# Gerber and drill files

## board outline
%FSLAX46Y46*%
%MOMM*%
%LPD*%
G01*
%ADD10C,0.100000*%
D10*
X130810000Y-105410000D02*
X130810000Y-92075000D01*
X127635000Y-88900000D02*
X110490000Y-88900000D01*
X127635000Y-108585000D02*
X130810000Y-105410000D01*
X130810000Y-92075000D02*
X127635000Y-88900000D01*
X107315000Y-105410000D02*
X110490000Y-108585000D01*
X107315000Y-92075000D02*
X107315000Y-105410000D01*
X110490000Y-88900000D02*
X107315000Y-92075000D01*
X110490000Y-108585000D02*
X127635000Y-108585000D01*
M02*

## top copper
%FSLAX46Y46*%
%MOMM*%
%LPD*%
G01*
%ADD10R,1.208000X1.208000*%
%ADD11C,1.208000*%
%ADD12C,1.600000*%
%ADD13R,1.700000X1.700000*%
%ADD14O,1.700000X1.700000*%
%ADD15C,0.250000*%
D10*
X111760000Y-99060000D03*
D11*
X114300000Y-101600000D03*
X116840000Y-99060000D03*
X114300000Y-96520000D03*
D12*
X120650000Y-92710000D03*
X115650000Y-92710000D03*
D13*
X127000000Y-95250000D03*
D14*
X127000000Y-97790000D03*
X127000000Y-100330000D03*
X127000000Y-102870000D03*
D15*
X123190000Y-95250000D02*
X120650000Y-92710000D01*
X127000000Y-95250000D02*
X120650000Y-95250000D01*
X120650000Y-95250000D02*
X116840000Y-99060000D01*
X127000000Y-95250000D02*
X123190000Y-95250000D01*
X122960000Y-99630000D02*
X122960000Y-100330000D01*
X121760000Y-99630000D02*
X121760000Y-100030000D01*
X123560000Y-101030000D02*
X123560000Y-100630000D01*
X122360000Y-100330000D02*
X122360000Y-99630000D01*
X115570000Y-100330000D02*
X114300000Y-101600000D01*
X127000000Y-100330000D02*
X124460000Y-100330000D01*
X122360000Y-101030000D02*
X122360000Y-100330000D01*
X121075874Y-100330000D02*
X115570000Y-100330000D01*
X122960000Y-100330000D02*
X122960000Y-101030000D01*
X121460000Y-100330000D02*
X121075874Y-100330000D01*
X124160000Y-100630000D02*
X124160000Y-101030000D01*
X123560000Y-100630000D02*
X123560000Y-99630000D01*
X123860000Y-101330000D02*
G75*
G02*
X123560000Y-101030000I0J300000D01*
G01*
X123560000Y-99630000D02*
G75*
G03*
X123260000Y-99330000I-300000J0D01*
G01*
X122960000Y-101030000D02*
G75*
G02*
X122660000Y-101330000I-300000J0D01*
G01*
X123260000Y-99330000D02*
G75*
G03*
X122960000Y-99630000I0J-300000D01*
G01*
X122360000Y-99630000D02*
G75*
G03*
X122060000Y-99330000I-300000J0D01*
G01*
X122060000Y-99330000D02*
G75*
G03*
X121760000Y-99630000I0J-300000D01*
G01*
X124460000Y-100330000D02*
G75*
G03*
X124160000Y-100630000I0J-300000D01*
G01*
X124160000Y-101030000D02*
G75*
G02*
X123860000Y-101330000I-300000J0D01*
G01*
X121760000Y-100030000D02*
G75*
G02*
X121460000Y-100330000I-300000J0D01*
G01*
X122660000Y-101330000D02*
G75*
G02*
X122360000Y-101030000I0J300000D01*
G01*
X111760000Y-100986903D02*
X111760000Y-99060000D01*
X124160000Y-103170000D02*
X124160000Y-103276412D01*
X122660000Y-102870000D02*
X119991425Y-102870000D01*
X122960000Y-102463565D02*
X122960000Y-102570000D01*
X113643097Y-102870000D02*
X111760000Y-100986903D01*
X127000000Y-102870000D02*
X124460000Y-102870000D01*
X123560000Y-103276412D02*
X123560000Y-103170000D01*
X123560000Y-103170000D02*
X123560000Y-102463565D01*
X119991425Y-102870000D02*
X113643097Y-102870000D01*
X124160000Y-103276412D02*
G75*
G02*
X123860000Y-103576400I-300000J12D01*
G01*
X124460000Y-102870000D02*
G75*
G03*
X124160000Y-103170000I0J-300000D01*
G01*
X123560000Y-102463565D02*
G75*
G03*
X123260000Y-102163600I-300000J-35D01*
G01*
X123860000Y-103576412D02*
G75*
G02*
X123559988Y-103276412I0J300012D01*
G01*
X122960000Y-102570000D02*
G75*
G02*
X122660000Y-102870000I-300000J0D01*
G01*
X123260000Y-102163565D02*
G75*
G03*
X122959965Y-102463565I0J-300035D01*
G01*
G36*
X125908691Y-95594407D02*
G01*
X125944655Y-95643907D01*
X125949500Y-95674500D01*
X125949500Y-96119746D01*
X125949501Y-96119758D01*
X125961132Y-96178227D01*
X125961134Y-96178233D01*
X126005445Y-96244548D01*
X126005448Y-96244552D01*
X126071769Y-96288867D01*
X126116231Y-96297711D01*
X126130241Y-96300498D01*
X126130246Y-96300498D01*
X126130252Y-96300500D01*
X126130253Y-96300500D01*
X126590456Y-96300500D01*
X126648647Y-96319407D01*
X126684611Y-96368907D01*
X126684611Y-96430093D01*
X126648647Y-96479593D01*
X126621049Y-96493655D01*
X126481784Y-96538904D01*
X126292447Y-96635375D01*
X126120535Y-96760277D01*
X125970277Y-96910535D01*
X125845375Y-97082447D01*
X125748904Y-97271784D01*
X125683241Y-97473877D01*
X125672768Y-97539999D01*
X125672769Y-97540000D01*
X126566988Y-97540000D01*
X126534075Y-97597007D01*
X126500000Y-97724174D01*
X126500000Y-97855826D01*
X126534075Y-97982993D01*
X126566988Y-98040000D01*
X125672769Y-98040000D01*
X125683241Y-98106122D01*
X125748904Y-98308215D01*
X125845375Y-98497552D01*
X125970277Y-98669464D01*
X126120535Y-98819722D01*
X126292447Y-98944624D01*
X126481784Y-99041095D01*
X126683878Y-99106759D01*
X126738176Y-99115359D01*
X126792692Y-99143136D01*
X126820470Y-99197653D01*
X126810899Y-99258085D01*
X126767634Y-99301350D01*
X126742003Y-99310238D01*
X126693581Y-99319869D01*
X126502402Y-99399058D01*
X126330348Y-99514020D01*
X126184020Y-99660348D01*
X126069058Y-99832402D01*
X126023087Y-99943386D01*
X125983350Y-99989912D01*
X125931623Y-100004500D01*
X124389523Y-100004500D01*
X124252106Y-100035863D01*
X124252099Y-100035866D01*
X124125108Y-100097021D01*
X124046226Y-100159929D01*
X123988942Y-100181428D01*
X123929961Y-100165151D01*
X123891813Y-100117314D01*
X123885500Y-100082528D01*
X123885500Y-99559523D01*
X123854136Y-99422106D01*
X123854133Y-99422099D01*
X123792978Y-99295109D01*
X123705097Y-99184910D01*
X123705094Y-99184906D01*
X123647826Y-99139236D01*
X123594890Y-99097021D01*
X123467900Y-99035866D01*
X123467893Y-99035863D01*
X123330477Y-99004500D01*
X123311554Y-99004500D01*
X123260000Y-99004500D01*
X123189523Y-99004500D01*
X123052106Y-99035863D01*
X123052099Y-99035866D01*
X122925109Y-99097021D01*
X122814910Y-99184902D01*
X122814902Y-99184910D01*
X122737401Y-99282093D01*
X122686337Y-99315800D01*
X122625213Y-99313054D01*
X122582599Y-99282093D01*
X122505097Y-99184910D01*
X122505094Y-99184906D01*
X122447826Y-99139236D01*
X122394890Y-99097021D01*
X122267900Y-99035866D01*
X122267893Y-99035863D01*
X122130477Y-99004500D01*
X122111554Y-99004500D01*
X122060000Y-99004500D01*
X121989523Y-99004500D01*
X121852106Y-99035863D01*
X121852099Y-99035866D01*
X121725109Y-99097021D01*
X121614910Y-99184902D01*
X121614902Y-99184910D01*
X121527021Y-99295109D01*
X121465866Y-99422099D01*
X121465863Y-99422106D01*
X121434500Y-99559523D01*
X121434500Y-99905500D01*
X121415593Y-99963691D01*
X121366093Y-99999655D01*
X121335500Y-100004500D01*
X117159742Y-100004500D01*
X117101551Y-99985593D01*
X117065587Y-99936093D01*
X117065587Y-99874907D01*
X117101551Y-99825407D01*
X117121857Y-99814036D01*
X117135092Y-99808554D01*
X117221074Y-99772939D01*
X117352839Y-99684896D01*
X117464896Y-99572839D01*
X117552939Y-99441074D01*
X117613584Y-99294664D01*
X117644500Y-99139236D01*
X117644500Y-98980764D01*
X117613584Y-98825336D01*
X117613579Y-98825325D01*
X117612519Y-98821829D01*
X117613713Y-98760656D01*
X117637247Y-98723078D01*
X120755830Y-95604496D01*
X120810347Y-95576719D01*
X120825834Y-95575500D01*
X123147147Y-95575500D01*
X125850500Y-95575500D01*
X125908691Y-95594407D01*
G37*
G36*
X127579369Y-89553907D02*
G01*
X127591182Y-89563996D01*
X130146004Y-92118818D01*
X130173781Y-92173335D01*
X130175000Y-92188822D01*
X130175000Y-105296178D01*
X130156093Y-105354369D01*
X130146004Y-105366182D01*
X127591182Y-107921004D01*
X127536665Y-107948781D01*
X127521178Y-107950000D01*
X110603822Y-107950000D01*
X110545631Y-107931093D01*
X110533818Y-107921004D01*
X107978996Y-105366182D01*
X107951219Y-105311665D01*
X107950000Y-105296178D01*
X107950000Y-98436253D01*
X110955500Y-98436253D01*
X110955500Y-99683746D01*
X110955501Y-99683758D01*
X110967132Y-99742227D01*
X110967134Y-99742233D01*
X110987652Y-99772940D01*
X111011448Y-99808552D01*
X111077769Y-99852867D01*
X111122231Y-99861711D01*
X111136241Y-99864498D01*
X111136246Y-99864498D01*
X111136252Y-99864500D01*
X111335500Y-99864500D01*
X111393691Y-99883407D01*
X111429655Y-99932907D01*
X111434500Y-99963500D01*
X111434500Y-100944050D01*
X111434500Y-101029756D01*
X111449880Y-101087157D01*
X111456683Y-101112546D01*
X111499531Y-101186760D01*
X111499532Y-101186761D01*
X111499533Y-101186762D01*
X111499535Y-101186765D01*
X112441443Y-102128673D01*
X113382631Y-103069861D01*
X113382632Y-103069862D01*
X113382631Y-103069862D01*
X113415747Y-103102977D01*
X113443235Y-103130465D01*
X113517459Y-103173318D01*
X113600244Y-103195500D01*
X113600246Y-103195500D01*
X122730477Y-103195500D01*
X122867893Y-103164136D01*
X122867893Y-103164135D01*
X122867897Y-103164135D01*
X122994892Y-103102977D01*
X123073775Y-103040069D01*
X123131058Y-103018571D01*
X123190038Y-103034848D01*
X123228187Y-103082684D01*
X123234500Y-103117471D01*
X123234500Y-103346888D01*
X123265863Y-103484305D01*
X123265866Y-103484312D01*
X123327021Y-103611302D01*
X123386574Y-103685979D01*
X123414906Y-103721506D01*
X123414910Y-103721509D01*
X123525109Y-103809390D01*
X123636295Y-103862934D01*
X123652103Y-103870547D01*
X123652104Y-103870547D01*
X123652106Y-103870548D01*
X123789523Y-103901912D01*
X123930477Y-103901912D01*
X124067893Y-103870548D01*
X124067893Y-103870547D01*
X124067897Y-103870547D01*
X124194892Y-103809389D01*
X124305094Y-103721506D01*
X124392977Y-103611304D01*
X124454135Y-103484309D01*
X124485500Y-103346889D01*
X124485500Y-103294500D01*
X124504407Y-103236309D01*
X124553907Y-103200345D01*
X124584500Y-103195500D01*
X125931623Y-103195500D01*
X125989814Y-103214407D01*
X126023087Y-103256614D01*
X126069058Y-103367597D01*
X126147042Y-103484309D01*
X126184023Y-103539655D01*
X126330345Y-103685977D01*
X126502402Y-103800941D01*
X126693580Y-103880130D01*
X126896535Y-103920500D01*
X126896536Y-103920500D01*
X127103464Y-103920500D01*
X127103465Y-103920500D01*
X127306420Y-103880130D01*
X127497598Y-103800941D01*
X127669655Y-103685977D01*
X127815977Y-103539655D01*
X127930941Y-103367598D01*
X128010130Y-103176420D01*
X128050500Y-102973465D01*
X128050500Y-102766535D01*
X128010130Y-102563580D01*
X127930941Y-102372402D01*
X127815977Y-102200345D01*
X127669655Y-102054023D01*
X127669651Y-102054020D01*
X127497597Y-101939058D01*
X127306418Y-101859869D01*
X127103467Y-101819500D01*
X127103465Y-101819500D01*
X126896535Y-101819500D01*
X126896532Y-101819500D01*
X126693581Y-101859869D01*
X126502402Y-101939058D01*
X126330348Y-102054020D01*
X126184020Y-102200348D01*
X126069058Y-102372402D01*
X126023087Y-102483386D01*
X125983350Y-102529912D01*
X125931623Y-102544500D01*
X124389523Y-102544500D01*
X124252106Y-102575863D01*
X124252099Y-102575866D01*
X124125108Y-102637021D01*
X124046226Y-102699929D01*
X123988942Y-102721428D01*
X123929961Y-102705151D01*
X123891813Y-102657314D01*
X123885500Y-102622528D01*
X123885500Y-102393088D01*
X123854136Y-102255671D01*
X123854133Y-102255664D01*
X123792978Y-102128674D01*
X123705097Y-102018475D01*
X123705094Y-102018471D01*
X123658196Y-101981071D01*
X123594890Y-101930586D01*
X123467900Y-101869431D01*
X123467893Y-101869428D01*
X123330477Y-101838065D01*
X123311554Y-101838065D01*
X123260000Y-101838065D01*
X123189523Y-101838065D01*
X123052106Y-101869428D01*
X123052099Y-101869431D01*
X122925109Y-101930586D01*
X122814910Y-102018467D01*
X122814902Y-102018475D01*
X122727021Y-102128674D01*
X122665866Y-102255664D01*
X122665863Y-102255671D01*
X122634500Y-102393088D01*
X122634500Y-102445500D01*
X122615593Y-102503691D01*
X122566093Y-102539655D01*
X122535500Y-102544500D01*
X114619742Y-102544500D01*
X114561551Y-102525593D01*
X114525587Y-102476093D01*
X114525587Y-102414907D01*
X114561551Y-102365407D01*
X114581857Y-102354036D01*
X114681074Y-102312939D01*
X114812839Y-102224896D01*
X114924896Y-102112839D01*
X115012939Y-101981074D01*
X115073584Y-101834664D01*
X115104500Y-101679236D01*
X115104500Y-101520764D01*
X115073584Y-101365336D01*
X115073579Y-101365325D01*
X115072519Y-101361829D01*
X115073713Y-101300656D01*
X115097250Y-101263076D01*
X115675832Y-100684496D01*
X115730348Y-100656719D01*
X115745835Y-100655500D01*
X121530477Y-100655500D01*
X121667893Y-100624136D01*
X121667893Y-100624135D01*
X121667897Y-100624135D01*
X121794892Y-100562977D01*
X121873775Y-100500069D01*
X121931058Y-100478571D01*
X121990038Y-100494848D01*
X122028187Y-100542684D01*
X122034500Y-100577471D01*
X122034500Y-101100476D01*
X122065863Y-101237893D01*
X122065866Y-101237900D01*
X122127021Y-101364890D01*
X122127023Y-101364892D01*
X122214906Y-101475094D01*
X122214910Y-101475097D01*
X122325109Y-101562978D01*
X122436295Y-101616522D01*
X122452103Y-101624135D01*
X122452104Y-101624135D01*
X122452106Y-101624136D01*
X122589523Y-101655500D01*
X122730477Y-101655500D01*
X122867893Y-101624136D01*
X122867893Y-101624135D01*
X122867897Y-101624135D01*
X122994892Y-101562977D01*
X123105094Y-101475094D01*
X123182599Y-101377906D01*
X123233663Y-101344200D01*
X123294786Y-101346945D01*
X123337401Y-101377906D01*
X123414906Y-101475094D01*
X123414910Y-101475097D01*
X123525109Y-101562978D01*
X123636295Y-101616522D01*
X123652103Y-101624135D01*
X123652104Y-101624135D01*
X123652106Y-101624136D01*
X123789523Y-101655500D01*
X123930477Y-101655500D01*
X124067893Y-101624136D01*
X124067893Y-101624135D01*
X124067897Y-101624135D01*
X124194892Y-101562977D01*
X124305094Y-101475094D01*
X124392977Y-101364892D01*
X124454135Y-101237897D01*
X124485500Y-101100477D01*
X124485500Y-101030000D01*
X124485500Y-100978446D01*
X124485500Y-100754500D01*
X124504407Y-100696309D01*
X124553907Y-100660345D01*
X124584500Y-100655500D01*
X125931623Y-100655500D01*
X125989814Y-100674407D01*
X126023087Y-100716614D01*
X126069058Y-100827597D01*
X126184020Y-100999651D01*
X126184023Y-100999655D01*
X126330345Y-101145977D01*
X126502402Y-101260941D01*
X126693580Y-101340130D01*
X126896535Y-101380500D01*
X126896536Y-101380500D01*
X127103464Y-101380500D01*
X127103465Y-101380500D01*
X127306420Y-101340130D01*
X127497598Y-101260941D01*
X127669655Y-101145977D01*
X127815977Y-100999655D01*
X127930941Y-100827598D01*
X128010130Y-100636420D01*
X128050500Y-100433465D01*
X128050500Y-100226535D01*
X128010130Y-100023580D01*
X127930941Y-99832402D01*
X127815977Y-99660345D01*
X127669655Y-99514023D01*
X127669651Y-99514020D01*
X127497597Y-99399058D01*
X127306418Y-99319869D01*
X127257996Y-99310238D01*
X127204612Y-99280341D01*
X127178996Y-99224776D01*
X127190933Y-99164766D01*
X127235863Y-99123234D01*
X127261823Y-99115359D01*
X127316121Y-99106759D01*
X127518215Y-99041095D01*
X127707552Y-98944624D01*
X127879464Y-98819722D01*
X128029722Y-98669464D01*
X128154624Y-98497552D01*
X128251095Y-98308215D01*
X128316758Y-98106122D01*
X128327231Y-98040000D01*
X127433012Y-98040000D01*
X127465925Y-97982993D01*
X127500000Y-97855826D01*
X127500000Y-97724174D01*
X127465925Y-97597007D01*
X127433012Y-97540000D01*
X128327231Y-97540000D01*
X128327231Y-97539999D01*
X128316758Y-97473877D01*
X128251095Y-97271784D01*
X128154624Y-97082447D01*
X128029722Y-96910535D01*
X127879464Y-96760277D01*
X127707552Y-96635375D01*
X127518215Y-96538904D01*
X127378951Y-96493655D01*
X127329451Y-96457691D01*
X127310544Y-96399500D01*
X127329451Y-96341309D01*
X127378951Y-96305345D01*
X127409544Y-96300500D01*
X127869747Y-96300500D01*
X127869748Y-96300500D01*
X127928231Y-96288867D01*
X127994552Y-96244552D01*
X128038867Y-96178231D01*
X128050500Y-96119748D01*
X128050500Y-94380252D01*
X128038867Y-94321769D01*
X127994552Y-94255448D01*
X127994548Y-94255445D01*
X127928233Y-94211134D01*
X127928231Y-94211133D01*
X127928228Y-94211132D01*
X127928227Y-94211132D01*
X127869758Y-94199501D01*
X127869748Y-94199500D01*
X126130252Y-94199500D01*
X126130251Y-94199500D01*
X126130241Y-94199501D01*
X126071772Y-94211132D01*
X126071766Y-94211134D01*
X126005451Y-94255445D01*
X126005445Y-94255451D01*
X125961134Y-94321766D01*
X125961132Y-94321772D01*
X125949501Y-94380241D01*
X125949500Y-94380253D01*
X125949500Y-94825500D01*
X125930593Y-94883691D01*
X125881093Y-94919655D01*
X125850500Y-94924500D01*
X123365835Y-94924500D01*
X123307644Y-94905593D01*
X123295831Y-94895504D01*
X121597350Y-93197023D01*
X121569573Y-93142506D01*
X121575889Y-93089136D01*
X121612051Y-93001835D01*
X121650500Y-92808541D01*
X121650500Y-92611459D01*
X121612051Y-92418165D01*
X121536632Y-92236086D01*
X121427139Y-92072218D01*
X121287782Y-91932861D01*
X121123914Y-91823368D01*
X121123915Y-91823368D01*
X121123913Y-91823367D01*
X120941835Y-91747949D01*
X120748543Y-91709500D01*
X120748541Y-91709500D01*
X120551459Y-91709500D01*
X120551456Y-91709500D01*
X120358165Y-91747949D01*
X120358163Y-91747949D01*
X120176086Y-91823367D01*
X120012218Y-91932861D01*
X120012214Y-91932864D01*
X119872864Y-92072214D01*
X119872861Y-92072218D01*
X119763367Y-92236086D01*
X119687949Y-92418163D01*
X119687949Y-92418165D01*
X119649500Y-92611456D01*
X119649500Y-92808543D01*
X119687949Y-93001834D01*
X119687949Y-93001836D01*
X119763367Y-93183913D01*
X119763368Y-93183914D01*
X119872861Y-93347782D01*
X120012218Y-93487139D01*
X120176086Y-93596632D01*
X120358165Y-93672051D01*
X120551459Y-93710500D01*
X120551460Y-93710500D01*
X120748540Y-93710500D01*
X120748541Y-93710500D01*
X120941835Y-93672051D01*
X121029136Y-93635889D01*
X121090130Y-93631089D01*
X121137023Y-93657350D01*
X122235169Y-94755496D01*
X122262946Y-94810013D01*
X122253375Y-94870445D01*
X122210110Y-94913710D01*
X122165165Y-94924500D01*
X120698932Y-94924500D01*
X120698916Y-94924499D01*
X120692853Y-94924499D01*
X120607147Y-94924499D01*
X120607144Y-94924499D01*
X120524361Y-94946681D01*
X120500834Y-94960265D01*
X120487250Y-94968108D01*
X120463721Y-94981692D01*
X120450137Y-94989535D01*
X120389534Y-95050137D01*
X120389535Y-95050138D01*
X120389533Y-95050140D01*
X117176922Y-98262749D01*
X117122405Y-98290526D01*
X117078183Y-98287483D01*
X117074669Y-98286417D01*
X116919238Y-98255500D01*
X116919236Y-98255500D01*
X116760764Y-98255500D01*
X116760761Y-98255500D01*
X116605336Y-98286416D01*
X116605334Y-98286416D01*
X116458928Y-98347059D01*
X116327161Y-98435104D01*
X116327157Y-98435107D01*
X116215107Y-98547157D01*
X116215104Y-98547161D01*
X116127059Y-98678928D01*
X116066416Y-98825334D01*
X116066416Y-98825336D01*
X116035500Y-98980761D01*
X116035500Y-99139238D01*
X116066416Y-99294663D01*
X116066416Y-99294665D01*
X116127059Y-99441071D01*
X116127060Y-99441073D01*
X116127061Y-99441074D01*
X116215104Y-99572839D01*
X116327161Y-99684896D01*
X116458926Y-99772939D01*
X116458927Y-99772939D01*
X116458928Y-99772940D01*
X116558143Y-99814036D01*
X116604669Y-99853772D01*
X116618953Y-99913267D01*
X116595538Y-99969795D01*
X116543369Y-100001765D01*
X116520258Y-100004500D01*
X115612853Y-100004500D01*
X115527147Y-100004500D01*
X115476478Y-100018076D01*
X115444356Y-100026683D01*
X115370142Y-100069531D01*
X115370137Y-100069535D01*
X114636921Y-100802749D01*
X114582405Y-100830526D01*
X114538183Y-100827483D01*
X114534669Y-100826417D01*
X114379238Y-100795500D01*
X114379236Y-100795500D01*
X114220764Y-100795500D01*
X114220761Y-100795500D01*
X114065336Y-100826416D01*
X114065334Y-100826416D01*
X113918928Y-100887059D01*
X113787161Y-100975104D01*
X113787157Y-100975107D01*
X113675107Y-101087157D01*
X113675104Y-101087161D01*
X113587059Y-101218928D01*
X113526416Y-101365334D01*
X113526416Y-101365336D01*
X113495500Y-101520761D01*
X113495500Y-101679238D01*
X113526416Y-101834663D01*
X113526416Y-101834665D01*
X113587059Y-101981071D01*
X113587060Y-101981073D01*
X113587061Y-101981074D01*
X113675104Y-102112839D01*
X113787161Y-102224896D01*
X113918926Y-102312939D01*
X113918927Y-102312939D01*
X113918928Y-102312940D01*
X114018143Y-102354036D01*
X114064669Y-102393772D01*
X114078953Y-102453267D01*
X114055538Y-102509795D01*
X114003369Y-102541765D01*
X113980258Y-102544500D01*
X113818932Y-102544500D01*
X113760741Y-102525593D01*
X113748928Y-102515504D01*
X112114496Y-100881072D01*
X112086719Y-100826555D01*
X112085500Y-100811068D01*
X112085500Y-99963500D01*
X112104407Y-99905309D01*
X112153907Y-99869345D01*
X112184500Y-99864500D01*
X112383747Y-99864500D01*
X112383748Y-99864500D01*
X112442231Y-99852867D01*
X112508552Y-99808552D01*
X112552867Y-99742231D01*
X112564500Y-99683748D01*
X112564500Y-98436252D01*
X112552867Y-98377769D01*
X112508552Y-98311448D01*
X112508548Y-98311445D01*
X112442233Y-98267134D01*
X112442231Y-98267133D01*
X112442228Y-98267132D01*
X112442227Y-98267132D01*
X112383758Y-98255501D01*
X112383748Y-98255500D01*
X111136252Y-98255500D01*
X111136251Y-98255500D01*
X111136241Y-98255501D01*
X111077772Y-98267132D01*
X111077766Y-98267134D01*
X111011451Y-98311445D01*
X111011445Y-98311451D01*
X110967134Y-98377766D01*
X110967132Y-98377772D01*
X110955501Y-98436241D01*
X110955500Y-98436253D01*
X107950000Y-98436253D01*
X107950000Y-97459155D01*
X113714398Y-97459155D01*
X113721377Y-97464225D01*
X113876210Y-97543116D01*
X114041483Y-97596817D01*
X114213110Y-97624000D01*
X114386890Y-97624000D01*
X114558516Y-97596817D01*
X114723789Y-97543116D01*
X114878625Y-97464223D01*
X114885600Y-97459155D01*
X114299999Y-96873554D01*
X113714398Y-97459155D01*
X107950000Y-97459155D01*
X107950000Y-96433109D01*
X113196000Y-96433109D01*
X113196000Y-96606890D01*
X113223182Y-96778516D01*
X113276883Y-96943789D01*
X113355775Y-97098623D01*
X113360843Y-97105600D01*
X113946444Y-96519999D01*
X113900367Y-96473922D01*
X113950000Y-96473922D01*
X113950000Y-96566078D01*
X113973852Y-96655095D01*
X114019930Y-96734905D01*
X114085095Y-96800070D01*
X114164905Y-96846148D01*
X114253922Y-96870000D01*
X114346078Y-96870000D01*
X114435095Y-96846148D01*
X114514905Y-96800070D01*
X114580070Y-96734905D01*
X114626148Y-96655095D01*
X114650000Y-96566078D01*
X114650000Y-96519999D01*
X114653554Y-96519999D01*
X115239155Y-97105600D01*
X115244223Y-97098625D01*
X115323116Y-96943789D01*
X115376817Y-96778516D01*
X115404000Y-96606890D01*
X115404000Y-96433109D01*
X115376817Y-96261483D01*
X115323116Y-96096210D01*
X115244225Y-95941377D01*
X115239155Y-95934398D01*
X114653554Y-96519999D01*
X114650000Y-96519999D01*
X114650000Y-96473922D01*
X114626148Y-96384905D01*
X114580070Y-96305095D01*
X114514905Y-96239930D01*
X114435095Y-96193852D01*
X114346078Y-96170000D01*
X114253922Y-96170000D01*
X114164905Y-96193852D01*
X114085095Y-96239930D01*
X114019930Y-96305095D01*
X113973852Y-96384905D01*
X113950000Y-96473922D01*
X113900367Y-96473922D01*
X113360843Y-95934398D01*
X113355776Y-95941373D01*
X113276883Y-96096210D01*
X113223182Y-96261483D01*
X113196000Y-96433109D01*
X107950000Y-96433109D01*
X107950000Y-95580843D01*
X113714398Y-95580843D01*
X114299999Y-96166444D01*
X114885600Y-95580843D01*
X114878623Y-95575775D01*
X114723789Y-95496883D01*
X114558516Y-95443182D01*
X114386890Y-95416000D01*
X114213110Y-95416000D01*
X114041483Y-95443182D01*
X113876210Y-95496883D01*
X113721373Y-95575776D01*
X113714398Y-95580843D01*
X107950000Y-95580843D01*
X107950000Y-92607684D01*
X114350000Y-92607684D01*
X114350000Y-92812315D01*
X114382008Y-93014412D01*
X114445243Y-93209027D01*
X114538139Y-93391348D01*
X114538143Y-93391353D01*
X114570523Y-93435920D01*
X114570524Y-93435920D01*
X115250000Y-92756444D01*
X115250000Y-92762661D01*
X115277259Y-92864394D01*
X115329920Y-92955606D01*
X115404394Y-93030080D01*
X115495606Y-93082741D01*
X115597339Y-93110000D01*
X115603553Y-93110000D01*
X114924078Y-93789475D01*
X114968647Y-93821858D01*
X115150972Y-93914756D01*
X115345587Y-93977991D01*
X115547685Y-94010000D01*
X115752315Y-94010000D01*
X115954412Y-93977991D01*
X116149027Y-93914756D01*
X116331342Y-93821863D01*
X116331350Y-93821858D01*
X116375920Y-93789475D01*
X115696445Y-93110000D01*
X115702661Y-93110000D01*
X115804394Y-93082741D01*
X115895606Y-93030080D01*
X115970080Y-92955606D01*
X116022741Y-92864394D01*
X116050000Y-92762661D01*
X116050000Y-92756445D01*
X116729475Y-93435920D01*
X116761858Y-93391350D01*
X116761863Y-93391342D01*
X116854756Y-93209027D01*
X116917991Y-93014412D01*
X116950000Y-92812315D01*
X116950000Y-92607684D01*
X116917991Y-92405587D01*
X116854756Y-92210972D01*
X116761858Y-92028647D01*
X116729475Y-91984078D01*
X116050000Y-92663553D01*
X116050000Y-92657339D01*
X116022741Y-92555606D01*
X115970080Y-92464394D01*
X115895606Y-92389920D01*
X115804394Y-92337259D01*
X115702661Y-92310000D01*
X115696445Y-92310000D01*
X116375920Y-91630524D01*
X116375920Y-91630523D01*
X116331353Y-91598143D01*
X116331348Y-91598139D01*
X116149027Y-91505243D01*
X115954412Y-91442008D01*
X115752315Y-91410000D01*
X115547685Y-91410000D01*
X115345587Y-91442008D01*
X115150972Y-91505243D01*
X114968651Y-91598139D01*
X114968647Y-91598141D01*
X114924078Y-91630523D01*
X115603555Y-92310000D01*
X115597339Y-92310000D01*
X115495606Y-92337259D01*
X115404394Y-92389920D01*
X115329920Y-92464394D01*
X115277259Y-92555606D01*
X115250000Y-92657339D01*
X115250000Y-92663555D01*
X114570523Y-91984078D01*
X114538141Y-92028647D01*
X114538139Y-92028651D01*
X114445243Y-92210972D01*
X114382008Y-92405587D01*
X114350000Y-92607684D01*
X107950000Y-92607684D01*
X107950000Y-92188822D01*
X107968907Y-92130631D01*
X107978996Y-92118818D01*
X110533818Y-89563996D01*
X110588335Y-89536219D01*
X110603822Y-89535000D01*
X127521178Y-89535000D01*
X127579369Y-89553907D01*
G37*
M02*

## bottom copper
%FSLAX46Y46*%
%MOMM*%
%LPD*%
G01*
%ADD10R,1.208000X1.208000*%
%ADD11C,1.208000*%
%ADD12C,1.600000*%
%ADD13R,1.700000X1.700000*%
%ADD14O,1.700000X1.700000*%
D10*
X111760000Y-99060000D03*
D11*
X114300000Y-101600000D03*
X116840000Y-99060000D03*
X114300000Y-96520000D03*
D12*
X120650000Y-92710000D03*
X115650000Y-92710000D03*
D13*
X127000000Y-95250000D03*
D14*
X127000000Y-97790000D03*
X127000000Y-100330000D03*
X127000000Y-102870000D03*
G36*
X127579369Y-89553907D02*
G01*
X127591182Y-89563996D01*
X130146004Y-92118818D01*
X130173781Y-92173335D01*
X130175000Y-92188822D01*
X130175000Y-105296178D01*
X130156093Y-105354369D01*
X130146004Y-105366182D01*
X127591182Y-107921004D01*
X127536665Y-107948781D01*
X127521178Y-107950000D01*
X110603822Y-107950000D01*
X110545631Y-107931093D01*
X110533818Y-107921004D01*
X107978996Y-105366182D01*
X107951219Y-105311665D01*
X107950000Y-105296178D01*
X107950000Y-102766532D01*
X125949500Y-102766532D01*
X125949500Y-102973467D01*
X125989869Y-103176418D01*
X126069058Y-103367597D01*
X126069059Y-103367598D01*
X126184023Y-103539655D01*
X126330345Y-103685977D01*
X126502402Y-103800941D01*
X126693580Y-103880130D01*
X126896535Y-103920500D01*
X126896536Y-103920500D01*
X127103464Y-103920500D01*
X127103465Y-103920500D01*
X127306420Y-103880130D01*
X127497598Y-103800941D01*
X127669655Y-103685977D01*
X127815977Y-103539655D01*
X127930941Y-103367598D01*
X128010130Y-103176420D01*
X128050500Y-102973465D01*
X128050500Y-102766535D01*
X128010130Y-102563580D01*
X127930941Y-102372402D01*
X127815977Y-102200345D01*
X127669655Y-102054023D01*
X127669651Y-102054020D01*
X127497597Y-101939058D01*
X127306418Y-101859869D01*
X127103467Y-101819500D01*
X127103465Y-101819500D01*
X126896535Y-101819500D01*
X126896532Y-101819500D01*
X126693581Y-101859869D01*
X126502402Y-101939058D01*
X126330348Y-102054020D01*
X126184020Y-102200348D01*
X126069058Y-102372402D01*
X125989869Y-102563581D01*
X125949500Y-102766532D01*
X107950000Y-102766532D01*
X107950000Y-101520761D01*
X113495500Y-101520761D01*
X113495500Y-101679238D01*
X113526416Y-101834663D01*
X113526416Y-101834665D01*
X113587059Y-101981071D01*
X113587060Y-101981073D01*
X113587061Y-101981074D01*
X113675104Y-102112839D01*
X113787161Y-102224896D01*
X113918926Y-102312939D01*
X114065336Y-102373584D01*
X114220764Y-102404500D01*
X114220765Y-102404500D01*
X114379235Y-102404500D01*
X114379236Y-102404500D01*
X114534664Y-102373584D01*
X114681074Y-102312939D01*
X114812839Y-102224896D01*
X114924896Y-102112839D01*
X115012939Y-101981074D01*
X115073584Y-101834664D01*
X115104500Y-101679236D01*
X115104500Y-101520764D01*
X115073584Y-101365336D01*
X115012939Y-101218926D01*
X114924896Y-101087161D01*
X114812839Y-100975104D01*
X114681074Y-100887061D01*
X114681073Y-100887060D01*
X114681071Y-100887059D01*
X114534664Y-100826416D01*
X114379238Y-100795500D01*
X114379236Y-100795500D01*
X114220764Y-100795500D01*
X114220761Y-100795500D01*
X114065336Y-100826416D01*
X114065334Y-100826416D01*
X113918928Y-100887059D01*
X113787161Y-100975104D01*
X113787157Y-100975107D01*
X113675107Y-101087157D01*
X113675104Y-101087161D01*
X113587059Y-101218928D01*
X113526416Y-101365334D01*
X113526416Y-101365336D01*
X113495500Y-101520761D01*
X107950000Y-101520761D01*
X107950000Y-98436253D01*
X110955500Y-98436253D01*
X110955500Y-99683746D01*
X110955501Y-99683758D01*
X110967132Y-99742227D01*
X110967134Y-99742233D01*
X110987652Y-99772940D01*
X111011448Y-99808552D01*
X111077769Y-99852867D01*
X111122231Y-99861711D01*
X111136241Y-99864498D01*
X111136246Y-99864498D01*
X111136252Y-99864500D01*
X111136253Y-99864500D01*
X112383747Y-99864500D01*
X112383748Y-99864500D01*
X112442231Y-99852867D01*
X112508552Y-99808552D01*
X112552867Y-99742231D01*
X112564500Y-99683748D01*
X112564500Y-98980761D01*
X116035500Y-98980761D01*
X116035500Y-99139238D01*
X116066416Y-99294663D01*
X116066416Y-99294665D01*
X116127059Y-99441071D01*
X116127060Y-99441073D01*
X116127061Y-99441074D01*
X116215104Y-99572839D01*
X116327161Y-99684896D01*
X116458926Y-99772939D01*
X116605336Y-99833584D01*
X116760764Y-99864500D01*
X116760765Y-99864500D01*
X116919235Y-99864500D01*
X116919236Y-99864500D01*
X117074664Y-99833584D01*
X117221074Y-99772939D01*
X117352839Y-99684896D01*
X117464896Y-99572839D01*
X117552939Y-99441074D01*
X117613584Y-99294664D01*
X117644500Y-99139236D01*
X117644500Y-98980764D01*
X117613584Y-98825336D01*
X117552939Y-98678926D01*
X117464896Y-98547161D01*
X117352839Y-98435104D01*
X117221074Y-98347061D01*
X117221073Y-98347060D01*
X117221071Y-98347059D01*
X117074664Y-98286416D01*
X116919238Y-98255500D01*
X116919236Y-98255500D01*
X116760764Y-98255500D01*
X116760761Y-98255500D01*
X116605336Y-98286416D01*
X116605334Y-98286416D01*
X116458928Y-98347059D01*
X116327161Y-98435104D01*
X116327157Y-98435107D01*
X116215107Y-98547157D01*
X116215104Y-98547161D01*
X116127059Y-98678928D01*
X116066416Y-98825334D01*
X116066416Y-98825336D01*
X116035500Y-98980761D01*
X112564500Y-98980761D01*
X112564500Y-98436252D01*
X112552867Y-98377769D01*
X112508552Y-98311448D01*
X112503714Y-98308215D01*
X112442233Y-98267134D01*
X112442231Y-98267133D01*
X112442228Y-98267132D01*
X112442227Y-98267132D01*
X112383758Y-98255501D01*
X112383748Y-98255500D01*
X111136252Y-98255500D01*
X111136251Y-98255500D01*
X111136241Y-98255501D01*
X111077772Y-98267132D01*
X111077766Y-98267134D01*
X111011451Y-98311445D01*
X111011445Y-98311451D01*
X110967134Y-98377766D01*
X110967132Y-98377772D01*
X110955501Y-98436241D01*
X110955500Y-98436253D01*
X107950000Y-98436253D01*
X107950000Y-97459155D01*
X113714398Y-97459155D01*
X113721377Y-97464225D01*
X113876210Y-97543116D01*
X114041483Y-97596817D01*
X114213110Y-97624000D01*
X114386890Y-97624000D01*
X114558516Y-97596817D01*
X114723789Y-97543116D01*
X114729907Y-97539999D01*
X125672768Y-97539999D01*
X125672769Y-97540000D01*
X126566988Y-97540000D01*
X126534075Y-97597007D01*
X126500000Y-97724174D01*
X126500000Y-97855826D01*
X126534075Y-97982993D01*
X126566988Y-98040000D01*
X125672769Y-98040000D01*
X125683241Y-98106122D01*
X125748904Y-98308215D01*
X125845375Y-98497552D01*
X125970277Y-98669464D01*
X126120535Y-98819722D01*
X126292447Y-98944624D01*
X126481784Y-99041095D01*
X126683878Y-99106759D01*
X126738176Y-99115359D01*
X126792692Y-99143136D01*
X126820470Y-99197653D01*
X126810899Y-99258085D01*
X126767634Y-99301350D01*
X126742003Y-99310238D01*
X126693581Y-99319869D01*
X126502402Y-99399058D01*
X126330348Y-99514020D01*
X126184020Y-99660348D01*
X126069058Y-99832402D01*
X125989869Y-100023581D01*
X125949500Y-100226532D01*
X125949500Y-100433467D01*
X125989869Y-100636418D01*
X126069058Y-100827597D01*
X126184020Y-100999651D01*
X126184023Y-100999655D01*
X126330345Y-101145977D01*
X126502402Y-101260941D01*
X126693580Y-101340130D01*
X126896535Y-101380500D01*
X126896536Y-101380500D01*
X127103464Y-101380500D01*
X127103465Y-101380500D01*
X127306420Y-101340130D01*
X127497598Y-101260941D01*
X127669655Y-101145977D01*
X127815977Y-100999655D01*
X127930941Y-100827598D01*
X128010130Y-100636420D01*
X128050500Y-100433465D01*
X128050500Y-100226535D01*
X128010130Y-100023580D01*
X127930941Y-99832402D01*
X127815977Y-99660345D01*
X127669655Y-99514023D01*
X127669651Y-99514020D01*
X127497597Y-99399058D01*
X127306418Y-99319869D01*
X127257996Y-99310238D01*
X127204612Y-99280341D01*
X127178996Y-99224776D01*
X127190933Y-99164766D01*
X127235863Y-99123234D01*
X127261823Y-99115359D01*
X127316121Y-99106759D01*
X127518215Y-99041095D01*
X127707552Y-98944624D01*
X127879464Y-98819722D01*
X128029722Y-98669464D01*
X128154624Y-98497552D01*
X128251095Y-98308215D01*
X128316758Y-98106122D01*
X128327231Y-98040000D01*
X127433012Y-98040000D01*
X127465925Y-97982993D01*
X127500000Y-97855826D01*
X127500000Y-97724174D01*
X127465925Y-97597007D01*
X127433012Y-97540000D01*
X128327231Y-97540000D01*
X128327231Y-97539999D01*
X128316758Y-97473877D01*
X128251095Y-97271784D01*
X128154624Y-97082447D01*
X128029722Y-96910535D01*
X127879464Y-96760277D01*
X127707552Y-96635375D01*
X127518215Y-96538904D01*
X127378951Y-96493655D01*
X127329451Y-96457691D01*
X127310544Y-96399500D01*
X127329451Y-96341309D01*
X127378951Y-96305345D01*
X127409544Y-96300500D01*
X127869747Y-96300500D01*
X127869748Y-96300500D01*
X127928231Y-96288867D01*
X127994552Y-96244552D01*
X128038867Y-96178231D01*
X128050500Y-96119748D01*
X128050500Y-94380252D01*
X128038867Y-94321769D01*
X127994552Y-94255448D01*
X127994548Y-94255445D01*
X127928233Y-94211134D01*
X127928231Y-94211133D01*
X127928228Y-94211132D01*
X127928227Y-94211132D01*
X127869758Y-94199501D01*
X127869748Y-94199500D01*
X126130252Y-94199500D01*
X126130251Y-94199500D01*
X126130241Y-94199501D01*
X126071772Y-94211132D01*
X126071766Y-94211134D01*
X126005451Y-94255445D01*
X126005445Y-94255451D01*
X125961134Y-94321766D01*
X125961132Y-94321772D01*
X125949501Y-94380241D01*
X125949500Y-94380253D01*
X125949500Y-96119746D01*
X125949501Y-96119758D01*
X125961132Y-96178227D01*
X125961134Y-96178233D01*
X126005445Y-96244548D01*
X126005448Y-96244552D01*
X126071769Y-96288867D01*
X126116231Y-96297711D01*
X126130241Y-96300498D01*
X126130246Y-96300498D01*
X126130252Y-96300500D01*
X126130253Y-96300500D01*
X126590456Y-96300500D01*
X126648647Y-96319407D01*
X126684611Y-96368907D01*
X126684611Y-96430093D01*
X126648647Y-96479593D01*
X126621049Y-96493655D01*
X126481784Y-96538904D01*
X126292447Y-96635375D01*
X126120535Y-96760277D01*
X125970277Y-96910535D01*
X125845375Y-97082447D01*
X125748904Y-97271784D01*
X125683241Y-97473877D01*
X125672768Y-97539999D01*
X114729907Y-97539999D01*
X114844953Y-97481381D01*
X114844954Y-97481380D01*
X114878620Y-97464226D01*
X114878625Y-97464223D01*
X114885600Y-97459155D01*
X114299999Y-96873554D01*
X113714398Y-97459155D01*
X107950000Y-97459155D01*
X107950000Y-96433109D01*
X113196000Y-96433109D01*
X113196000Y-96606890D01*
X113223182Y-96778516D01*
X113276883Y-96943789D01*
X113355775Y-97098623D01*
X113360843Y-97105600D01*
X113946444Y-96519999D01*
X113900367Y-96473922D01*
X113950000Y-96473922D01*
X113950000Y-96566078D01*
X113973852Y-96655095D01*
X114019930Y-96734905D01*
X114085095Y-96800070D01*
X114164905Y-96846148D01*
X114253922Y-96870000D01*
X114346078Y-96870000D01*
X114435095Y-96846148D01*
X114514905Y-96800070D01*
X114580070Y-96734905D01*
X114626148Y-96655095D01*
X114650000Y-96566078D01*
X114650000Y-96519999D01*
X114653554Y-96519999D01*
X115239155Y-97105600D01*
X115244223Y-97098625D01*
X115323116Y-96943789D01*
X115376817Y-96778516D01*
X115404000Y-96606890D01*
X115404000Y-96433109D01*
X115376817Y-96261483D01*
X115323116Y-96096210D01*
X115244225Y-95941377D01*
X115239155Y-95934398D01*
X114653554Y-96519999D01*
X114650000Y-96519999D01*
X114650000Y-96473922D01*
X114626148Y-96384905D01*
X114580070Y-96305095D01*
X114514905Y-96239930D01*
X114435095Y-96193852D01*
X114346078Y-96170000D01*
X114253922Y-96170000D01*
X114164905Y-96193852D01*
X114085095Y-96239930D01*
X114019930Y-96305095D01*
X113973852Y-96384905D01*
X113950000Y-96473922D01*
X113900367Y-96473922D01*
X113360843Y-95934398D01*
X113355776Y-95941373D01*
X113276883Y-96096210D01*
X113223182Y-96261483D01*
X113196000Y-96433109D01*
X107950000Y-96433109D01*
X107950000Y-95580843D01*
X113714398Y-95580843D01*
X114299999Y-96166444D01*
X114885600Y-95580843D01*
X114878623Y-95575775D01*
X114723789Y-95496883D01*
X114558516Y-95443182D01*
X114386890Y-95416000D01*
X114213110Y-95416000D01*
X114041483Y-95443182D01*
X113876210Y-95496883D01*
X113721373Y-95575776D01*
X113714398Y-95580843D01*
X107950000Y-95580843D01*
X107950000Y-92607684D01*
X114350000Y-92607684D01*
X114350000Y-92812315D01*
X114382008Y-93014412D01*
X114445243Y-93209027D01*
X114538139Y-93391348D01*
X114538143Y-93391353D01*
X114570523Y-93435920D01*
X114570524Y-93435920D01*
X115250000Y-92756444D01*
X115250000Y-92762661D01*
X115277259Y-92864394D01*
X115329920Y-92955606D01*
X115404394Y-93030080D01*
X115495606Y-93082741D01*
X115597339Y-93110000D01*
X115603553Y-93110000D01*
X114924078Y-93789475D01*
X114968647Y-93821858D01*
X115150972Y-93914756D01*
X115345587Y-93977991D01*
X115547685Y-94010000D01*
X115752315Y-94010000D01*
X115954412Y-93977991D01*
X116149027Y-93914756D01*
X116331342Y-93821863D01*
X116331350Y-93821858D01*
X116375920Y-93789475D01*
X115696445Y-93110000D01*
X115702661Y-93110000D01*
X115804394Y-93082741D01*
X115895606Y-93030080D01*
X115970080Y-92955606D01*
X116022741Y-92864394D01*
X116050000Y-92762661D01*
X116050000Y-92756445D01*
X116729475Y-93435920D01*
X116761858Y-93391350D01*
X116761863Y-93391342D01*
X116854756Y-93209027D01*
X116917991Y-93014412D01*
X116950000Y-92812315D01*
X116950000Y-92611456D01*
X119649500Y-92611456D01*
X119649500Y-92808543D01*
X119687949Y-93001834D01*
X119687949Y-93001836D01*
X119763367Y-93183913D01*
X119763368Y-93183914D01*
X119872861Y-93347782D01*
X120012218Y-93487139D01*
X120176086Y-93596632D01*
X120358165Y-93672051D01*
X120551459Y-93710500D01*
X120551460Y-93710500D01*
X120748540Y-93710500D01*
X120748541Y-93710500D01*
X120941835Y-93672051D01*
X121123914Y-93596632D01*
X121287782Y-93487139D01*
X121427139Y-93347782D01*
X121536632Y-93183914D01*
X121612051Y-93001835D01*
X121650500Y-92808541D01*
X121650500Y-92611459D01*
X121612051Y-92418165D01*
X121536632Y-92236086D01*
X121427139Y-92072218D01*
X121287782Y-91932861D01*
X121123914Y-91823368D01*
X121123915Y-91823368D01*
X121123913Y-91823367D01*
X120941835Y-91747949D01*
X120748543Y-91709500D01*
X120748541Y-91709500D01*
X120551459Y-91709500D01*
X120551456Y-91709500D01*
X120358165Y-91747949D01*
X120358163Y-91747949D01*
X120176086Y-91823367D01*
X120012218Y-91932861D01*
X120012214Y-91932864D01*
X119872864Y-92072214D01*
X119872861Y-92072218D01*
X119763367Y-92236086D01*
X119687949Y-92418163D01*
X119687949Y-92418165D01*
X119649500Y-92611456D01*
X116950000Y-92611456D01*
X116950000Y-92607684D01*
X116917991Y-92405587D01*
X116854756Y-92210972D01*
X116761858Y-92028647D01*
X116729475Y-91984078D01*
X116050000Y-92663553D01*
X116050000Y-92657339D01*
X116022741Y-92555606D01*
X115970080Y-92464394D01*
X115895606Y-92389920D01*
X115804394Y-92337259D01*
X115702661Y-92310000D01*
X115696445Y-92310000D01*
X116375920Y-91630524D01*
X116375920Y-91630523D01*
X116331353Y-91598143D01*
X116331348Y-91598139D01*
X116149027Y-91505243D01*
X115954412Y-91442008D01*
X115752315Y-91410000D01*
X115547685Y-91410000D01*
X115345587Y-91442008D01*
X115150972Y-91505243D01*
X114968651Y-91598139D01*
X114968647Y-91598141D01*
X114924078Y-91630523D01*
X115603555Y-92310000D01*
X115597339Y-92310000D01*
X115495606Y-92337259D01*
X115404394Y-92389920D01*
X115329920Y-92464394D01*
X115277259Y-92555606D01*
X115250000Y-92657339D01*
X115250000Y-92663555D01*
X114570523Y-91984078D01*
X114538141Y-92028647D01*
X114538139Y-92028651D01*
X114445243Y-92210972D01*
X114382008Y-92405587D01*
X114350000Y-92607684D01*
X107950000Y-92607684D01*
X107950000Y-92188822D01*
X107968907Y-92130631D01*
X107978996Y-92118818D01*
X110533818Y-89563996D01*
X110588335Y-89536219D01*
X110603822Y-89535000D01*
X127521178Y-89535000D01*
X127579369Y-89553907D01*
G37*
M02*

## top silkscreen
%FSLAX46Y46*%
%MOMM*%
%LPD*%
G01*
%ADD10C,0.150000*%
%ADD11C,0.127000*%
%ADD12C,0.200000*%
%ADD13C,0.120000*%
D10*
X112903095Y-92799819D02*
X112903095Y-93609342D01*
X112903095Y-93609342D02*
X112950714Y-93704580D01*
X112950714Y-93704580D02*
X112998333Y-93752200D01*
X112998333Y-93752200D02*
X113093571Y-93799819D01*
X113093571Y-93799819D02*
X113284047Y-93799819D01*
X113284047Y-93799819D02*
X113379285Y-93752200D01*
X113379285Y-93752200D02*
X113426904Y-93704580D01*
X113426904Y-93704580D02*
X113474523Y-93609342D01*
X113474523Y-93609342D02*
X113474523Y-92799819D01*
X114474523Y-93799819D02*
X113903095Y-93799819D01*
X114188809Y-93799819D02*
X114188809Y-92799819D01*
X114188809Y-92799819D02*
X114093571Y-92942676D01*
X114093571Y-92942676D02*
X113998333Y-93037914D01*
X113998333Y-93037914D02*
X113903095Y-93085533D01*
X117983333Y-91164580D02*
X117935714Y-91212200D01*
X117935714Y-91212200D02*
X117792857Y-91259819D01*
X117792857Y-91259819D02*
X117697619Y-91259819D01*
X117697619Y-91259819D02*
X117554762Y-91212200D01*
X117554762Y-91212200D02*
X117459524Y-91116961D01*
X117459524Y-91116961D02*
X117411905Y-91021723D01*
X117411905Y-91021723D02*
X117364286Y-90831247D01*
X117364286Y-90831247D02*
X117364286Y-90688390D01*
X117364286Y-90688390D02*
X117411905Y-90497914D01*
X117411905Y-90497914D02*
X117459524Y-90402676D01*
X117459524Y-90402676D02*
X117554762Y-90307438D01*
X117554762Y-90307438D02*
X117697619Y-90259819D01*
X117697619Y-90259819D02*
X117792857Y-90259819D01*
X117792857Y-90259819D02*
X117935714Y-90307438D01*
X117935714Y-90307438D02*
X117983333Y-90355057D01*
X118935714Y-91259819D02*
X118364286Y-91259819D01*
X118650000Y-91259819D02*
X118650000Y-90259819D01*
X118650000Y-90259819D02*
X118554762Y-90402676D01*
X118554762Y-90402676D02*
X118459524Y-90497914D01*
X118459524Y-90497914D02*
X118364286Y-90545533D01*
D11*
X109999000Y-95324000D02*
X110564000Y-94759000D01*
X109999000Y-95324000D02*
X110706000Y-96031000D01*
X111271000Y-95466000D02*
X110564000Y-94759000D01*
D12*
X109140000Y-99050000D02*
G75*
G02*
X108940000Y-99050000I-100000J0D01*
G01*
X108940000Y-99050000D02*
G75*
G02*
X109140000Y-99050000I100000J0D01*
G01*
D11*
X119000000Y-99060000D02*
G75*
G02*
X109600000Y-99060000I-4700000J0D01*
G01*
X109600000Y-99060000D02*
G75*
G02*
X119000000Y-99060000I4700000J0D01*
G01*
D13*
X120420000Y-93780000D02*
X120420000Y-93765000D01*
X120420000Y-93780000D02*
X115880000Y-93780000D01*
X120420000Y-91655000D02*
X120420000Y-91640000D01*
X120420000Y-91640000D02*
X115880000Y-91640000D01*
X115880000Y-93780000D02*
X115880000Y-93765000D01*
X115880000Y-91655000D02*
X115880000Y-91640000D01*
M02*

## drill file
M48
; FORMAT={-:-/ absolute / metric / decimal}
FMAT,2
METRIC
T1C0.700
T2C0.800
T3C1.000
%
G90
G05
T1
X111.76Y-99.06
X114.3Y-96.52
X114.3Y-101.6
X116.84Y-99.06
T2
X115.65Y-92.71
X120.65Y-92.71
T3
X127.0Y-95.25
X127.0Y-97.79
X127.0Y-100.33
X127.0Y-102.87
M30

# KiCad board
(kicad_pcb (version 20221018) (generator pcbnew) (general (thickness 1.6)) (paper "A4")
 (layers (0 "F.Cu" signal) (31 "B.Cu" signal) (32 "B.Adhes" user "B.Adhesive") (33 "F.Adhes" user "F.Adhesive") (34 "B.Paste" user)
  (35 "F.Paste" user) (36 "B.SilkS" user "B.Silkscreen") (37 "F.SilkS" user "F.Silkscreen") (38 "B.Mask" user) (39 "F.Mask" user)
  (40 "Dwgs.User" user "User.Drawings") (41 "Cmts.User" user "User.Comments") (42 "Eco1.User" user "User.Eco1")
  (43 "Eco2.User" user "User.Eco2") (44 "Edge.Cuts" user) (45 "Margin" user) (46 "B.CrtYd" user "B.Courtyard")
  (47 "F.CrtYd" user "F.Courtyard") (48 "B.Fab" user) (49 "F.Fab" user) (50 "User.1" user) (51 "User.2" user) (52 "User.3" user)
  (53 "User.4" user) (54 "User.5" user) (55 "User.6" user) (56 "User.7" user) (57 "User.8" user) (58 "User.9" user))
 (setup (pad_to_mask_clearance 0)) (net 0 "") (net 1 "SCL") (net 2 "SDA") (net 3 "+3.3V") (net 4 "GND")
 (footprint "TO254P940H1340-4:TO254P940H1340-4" (layer "F.Cu") (at 114.3 99.06)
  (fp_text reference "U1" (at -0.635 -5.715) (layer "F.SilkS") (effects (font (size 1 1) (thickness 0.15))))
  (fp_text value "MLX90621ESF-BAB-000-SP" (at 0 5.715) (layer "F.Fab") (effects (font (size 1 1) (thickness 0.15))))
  (fp_line (start -4.301 -3.736) (end -3.736 -4.301) (stroke (width 0.127) (type solid)) (layer "F.SilkS"))
  (fp_line (start -4.301 -3.736) (end -3.594 -3.029) (stroke (width 0.127) (type solid)) (layer "F.SilkS"))
  (fp_line (start -3.029 -3.594) (end -3.736 -4.301) (stroke (width 0.127) (type solid)) (layer "F.SilkS"))
  (fp_circle (center -5.26 -0.01) (end -5.16 -0.01) (stroke (width 0.2) (type solid)) (fill none) (layer "F.SilkS"))
  (fp_circle (center 0 0) (end 4.7 0) (stroke (width 0.127) (type solid)) (fill none) (layer "F.SilkS"))
  (pad "1" thru_hole rect (at -2.54 0) (size 1.208 1.208) (drill 0.7) (layers "*.Cu" "*.Mask") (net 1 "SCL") (solder_mask_margin 0.102))
  (pad "2" thru_hole circle (at 0 2.54) (size 1.208 1.208) (drill 0.7) (layers "*.Cu" "*.Mask") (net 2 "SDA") (solder_mask_margin 0.102))
  (pad "3" thru_hole circle (at 2.54 0) (size 1.208 1.208) (drill 0.7) (layers "*.Cu" "*.Mask") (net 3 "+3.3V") (solder_mask_margin 0.102))
  (pad "4" thru_hole circle (at 0 -2.54) (size 1.208 1.208) (drill 0.7) (layers "*.Cu" "*.Mask") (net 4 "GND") (solder_mask_margin 0.102)))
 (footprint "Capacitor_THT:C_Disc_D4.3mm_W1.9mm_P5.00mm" (layer "F.Cu") (at 120.65 92.71 180)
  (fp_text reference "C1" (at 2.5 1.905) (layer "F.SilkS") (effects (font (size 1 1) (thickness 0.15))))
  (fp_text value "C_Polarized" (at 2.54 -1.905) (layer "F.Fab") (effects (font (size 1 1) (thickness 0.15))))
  (fp_line (start 0.23 -1.07) (end 0.23 -1.055) (stroke (width 0.12) (type solid)) (layer "F.SilkS"))
  (fp_line (start 0.23 -1.07) (end 4.77 -1.07) (stroke (width 0.12) (type solid)) (layer "F.SilkS"))
  (fp_line (start 0.23 1.055) (end 0.23 1.07) (stroke (width 0.12) (type solid)) (layer "F.SilkS"))
  (fp_line (start 0.23 1.07) (end 4.77 1.07) (stroke (width 0.12) (type solid)) (layer "F.SilkS"))
  (fp_line (start 4.77 -1.07) (end 4.77 -1.055) (stroke (width 0.12) (type solid)) (layer "F.SilkS"))
  (fp_line (start 4.77 1.055) (end 4.77 1.07) (stroke (width 0.12) (type solid)) (layer "F.SilkS"))
  (pad "1" thru_hole circle (at 0 0 180) (size 1.6 1.6) (drill 0.8) (layers "*.Cu" "*.Mask") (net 3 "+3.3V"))
  (pad "2" thru_hole circle (at 5 0 180) (size 1.6 1.6) (drill 0.8) (layers "*.Cu" "*.Mask") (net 4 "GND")))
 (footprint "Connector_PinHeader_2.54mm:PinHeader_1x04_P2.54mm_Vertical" (layer "B.Cu") (at 127 95.25 180)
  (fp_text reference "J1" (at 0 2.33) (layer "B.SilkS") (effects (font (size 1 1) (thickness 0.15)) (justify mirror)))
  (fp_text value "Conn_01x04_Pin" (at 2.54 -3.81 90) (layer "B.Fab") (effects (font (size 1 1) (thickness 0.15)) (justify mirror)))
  (pad "1" thru_hole rect (at 0 0 180) (size 1.7 1.7) (drill 1) (layers "*.Cu" "*.Mask") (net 3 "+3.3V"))
  (pad "2" thru_hole oval (at 0 -2.54 180) (size 1.7 1.7) (drill 1) (layers "*.Cu" "*.Mask") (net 4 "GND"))
  (pad "3" thru_hole oval (at 0 -5.08 180) (size 1.7 1.7) (drill 1) (layers "*.Cu" "*.Mask") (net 2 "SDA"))
  (pad "4" thru_hole oval (at 0 -7.62 180) (size 1.7 1.7) (drill 1) (layers "*.Cu" "*.Mask") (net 1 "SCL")))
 (gr_line (start 130.81 105.41) (end 130.81 92.075) (stroke (width 0.1) (type default)) (layer "Edge.Cuts"))
 (gr_line (start 127.635 88.9) (end 110.49 88.9) (stroke (width 0.1) (type default)) (layer "Edge.Cuts"))
 (gr_line (start 127.635 108.585) (end 130.81 105.41) (stroke (width 0.1) (type default)) (layer "Edge.Cuts"))
 (gr_line (start 130.81 92.075) (end 127.635 88.9) (stroke (width 0.1) (type default)) (layer "Edge.Cuts"))
 (gr_line (start 107.315 105.41) (end 110.49 108.585) (stroke (width 0.1) (type default)) (layer "Edge.Cuts"))
 (gr_line (start 107.315 92.075) (end 107.315 105.41) (stroke (width 0.1) (type default)) (layer "Edge.Cuts"))
 (gr_line (start 110.49 88.9) (end 107.315 92.075) (stroke (width 0.1) (type default)) (layer "Edge.Cuts"))
 (gr_line (start 110.49 108.585) (end 127.635 108.585) (stroke (width 0.1) (type default)) (layer "Edge.Cuts"))
 (segment (start 123.19 95.25) (end 120.65 92.71) (width 0.25) (layer "F.Cu") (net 3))
 (segment (start 127 95.25) (end 120.65 95.25) (width 0.25) (layer "F.Cu") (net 3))
 (segment (start 120.65 95.25) (end 116.84 99.06) (width 0.25) (layer "F.Cu") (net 3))
 (segment (start 127 95.25) (end 123.19 95.25) (width 0.25) (layer "F.Cu") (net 3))
 (segment (start 122.96 99.63) (end 122.96 100.33) (width 0.25) (layer "F.Cu") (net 2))
 (segment (start 121.76 99.63) (end 121.76 100.03) (width 0.25) (layer "F.Cu") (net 2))
 (segment (start 123.56 101.03) (end 123.56 100.63) (width 0.25) (layer "F.Cu") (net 2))
 (segment (start 122.36 100.33) (end 122.36 99.63) (width 0.25) (layer "F.Cu") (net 2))
 (segment (start 115.57 100.33) (end 114.3 101.6) (width 0.25) (layer "F.Cu") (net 2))
 (segment (start 127 100.33) (end 124.46 100.33) (width 0.25) (layer "F.Cu") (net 2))
 (segment (start 122.36 101.03) (end 122.36 100.33) (width 0.25) (layer "F.Cu") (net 2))
 (segment (start 121.075874 100.33) (end 115.57 100.33) (width 0.25) (layer "F.Cu") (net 2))
 (segment (start 122.96 100.33) (end 122.96 101.03) (width 0.25) (layer "F.Cu") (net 2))
 (segment (start 121.46 100.33) (end 121.075874 100.33) (width 0.25) (layer "F.Cu") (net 2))
 (segment (start 124.16 100.63) (end 124.16 101.03) (width 0.25) (layer "F.Cu") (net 2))
 (segment (start 123.56 100.63) (end 123.56 99.63) (width 0.25) (layer "F.Cu") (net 2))
 (arc (start 123.86 101.33) (mid 123.647868 101.242132) (end 123.56 101.03) (width 0.25) (layer "F.Cu") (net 2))
 (arc (start 123.56 99.63) (mid 123.472132 99.417868) (end 123.26 99.33) (width 0.25) (layer "F.Cu") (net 2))
 (arc (start 122.96 101.03) (mid 122.872132 101.242132) (end 122.66 101.33) (width 0.25) (layer "F.Cu") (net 2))
 (arc (start 123.26 99.33) (mid 123.047868 99.417868) (end 122.96 99.63) (width 0.25) (layer "F.Cu") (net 2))
 (arc (start 122.36 99.63) (mid 122.272132 99.417868) (end 122.06 99.33) (width 0.25) (layer "F.Cu") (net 2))
 (arc (start 122.06 99.33) (mid 121.847868 99.417868) (end 121.76 99.63) (width 0.25) (layer "F.Cu") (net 2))
 (arc (start 124.46 100.33) (mid 124.247868 100.417868) (end 124.16 100.63) (width 0.25) (layer "F.Cu") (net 2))
 (arc (start 124.16 101.03) (mid 124.072132 101.242132) (end 123.86 101.33) (width 0.25) (layer "F.Cu") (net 2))
 (arc (start 121.76 100.03) (mid 121.672132 100.242132) (end 121.46 100.33) (width 0.25) (layer "F.Cu") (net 2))
 (arc (start 122.66 101.33) (mid 122.447868 101.242132) (end 122.36 101.03) (width 0.25) (layer "F.Cu") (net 2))
 (segment (start 111.76 100.986903) (end 111.76 99.06) (width 0.25) (layer "F.Cu") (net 1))
 (segment (start 124.16 103.17) (end 124.16 103.276412) (width 0.25) (layer "F.Cu") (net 1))
 (segment (start 122.66 102.87) (end 119.991425 102.87) (width 0.25) (layer "F.Cu") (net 1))
 (segment (start 122.96 102.463565) (end 122.96 102.57) (width 0.25) (layer "F.Cu") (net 1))
 (segment (start 113.643097 102.87) (end 111.76 100.986903) (width 0.25) (layer "F.Cu") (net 1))
 (segment (start 127 102.87) (end 124.46 102.87) (width 0.25) (layer "F.Cu") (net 1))
 (segment (start 123.56 103.276412) (end 123.56 103.17) (width 0.25) (layer "F.Cu") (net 1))
 (segment (start 123.56 103.17) (end 123.56 102.463565) (width 0.25) (layer "F.Cu") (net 1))
 (segment (start 119.991425 102.87) (end 113.643097 102.87) (width 0.25) (layer "F.Cu") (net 1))
 (arc (start 124.16 103.276412) (mid 124.072132 103.488544) (end 123.86 103.576412) (width 0.25) (layer "F.Cu") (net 1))
 (arc (start 124.46 102.87) (mid 124.247868 102.957868) (end 124.16 103.17) (width 0.25) (layer "F.Cu") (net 1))
 (arc (start 123.56 102.463565) (mid 123.472132 102.251433) (end 123.26 102.163565) (width 0.25) (layer "F.Cu") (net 1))
 (arc (start 123.86 103.576412) (mid 123.647868 103.488544) (end 123.56 103.276412) (width 0.25) (layer "F.Cu") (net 1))
 (arc (start 122.96 102.57) (mid 122.872132 102.782132) (end 122.66 102.87) (width 0.25) (layer "F.Cu") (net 1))
 (arc (start 123.26 102.163565) (mid 123.047868 102.251433) (end 122.96 102.463565) (width 0.25) (layer "F.Cu") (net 1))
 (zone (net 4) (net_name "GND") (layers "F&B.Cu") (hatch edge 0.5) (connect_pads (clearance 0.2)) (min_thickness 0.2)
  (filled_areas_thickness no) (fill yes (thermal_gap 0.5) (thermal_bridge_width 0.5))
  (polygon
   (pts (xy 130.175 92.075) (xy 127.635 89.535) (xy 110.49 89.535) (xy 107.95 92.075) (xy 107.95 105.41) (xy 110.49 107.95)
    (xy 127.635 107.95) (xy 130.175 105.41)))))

